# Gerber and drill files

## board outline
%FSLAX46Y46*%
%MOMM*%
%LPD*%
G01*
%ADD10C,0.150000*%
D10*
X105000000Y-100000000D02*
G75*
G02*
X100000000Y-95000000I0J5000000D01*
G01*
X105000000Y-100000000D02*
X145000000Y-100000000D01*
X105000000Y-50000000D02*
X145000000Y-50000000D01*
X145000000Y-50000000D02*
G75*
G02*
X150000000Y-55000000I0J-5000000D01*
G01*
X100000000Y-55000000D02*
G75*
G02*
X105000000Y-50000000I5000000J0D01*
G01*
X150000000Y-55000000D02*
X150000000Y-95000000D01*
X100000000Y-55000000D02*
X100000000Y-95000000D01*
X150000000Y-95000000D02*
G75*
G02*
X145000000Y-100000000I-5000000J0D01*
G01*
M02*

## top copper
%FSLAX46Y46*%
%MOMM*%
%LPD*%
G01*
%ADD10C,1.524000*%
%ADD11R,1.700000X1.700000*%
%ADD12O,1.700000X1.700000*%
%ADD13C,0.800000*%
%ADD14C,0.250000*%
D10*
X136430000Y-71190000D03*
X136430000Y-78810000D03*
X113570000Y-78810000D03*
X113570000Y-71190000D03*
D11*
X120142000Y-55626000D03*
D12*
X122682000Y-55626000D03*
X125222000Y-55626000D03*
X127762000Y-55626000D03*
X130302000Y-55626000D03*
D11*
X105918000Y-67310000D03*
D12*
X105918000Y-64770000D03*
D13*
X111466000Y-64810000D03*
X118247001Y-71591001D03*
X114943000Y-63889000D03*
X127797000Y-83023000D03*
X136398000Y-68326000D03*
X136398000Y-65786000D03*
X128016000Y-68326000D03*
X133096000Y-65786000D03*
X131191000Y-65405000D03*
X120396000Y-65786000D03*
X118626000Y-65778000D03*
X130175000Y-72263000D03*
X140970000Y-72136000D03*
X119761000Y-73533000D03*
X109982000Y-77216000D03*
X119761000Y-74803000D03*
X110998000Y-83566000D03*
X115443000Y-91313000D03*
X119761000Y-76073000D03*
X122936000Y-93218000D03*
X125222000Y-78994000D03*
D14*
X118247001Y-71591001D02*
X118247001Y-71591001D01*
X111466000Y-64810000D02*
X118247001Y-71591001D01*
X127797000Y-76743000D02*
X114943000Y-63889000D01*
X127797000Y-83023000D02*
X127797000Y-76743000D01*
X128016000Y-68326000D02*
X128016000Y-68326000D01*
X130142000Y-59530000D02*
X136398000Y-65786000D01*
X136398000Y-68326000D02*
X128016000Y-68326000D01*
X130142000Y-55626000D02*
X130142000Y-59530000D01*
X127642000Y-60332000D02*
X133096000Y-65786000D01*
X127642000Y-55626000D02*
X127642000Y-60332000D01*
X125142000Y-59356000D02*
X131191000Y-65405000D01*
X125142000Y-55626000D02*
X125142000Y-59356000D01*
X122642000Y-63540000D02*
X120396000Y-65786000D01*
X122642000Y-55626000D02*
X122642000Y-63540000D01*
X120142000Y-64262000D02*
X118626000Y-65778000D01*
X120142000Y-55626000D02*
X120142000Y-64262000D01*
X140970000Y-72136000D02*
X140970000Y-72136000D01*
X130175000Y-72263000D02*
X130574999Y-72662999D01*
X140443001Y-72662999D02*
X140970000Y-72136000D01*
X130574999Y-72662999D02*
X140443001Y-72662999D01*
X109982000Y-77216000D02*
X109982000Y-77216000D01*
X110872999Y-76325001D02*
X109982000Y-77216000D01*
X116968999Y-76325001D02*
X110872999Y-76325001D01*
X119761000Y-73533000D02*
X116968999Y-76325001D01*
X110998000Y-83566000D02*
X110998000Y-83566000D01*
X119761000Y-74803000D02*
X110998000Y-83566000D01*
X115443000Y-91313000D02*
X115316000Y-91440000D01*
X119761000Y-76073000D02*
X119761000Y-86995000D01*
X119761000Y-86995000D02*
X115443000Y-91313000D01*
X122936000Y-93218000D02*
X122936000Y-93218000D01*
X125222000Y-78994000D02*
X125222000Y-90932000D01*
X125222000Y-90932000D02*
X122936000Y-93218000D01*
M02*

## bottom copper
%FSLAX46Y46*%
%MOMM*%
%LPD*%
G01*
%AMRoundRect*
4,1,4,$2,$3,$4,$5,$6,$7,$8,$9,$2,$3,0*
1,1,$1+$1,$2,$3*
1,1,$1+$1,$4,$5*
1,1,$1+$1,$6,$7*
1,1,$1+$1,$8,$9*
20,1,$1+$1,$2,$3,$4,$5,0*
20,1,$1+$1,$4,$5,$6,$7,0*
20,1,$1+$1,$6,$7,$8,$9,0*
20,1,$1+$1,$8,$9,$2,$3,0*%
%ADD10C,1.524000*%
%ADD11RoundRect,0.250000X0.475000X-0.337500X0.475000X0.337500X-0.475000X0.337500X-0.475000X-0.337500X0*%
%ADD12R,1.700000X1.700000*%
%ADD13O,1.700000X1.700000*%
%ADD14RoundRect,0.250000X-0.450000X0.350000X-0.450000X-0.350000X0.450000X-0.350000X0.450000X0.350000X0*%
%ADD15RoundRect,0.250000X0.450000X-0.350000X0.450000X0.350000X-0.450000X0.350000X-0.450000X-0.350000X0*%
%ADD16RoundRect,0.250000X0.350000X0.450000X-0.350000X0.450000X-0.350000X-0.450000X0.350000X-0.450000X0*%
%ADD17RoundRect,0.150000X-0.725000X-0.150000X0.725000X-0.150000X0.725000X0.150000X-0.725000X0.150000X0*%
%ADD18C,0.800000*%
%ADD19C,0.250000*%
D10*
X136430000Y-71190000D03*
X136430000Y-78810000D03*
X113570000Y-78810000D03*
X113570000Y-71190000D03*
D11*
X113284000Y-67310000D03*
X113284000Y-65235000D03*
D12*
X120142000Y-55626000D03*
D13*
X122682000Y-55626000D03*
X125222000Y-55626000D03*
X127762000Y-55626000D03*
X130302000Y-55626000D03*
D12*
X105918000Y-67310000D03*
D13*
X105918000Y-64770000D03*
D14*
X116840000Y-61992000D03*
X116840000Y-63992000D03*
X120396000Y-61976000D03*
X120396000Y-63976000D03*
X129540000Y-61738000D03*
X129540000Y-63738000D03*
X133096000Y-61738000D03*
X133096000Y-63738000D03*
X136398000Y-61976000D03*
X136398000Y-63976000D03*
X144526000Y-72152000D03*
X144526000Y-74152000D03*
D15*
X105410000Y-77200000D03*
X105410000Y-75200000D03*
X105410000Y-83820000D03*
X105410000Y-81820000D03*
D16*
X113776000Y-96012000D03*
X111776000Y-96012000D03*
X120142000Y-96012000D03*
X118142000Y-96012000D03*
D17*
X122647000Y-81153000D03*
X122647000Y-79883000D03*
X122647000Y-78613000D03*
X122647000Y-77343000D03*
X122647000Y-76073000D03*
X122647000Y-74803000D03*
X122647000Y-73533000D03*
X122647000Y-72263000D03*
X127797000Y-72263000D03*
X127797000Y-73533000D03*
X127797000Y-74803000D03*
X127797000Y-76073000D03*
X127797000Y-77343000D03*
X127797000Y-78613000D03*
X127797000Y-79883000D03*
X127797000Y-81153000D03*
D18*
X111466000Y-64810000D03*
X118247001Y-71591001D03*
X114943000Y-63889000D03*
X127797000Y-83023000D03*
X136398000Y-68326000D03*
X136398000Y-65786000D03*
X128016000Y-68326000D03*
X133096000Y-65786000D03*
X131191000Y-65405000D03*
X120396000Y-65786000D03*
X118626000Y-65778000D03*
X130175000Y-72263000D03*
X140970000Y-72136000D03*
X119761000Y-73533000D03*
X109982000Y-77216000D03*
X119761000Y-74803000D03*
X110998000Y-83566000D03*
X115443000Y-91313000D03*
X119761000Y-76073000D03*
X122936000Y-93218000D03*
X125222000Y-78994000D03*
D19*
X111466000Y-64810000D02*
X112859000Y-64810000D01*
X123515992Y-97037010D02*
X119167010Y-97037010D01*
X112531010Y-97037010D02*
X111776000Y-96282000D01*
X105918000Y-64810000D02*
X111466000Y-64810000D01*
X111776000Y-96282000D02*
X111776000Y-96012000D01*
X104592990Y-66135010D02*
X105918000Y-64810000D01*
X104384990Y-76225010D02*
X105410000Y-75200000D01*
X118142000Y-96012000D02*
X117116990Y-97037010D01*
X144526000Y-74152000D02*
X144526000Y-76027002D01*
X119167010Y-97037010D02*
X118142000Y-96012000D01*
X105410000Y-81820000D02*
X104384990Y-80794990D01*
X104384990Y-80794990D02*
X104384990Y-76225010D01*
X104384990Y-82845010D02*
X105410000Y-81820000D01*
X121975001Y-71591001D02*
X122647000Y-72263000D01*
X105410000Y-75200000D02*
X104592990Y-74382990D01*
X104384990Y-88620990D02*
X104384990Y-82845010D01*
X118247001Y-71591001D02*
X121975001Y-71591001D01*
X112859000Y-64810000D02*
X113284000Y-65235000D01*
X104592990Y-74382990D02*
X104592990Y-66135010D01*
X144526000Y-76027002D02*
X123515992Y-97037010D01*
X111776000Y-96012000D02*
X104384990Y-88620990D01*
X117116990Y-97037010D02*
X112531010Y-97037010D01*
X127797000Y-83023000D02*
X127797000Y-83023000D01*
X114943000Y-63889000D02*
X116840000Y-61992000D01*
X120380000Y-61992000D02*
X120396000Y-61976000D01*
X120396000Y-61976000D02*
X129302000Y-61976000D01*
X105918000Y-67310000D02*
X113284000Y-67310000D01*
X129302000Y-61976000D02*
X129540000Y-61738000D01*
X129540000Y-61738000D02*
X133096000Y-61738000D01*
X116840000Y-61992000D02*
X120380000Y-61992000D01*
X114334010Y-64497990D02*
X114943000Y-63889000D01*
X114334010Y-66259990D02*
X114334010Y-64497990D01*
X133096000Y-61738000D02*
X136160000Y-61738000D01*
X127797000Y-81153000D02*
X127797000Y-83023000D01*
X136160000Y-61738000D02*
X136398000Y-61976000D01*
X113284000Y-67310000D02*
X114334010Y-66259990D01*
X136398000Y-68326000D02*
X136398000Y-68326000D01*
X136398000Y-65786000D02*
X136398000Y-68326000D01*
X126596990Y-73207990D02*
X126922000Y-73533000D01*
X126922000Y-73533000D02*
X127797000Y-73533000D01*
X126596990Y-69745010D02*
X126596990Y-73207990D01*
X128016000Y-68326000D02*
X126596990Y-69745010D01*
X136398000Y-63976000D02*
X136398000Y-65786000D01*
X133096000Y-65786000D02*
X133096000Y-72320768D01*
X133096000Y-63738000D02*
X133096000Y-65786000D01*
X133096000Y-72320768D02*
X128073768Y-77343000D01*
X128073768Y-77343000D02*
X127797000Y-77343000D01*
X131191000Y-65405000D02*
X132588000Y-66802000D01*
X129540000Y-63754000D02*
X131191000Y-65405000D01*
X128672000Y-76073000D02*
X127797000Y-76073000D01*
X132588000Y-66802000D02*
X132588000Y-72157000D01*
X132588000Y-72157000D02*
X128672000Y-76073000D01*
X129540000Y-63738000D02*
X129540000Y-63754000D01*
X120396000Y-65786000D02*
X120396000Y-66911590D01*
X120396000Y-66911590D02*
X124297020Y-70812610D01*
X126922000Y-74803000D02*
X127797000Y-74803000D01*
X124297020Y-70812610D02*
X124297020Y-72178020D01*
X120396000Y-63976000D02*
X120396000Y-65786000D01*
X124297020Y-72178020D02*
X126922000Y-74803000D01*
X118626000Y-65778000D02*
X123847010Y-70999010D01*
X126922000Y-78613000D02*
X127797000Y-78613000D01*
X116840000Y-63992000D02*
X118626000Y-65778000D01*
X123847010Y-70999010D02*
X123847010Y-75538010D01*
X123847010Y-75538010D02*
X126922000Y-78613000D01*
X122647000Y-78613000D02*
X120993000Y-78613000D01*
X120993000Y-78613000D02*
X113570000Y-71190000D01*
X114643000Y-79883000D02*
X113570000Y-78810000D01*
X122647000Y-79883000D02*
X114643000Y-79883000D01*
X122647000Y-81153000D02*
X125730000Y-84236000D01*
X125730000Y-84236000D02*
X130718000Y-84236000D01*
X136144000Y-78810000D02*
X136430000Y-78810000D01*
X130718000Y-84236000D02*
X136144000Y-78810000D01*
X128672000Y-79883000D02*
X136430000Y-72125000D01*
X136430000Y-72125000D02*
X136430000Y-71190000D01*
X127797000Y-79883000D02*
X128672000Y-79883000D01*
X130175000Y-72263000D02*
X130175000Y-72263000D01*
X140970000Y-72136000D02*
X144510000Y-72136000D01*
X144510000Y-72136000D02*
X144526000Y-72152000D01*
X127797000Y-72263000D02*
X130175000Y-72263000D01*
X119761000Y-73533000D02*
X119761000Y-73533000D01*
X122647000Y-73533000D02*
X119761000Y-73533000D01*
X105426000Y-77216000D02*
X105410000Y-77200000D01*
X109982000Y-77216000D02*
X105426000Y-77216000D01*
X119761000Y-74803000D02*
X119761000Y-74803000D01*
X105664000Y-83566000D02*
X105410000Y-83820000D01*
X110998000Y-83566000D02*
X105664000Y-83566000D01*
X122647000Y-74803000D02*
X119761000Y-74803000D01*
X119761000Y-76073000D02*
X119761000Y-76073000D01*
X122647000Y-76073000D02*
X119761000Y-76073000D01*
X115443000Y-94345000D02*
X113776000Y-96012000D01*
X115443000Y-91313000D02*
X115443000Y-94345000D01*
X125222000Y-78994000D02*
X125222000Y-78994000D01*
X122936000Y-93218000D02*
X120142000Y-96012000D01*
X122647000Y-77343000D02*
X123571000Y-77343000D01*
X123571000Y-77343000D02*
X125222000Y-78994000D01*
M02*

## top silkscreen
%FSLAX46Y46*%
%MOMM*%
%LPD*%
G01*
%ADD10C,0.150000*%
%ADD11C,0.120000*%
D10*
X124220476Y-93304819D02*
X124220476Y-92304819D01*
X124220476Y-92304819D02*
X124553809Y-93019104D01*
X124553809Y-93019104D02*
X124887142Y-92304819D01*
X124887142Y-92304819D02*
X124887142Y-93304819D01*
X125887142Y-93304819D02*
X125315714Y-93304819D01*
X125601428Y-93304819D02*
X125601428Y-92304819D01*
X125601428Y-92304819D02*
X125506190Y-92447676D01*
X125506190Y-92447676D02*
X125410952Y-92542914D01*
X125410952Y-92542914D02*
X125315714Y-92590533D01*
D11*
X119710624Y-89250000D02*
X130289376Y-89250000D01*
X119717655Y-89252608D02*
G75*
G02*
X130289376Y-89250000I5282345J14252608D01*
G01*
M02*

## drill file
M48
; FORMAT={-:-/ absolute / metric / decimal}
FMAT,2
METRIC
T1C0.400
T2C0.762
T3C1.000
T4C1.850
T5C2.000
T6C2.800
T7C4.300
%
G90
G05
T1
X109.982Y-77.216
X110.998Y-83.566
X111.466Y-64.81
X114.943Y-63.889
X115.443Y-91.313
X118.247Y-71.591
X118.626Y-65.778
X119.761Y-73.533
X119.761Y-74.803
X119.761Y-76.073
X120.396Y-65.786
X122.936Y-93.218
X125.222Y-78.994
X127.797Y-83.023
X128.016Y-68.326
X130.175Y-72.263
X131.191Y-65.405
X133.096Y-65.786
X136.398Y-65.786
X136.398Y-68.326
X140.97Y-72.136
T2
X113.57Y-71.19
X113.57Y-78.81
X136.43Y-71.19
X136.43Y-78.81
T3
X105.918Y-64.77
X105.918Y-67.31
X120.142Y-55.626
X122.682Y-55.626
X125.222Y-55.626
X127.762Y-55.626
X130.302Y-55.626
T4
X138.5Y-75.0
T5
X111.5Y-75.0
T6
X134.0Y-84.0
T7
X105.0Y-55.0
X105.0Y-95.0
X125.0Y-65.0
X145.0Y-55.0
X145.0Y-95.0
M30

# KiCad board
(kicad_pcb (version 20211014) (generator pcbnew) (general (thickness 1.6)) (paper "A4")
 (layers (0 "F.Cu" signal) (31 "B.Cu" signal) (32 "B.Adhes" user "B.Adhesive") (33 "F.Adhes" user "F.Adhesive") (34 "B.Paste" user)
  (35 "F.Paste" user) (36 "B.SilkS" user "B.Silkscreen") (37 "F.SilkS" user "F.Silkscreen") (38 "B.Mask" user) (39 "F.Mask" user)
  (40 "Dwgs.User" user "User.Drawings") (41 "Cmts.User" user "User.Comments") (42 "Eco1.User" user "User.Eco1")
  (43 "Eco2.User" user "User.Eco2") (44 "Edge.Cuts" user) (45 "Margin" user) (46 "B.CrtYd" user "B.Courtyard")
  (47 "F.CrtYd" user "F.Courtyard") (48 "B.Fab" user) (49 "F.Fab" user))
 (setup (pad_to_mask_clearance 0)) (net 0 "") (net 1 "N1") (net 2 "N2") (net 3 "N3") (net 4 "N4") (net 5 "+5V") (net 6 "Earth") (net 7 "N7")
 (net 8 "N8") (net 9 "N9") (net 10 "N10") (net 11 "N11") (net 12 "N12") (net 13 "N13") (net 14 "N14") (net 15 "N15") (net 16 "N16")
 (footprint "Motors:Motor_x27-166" (layer "F.Cu") (at 125 75)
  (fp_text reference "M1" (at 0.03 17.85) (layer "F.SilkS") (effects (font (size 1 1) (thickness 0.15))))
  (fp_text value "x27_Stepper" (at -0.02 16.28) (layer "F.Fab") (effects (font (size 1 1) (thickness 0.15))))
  (fp_line (start -5.289376 14.25) (end 5.289376 14.25) (layer "F.SilkS") (width 0.12))
  (fp_arc (start -5.282345 14.252608) (mid -0.00375 -15.2) (end 5.289376 14.25) (layer "F.SilkS") (width 0.12))
  (pad "" np_thru_hole circle locked (at 13.5 0) (size 1.85 1.85) (drill 1.85) (layers *.Cu *.Mask))
  (pad "" np_thru_hole circle locked (at 0 -10) (size 4.3 4.3) (drill 4.3) (layers *.Cu *.Mask))
  (pad "" np_thru_hole circle locked (at 9 9) (size 2.8 2.8) (drill 2.8) (layers *.Cu *.Mask))
  (pad "" np_thru_hole circle locked (at -13.5 0) (size 2 2) (drill 2) (layers *.Cu *.Mask))
  (pad "1" thru_hole circle locked (at 11.43 -3.81) (size 1.524 1.524) (drill 0.762) (layers *.Cu *.Mask) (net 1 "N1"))
  (pad "2" thru_hole circle locked (at 11.43 3.81) (size 1.524 1.524) (drill 0.762) (layers *.Cu *.Mask) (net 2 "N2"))
  (pad "3" thru_hole circle locked (at -11.43 3.81) (size 1.524 1.524) (drill 0.762) (layers *.Cu *.Mask) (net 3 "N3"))
  (pad "4" thru_hole circle locked (at -11.43 -3.81) (size 1.524 1.524) (drill 0.762) (layers *.Cu *.Mask) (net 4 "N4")))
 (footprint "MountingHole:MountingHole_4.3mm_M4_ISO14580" (layer "F.Cu") (at 105 55)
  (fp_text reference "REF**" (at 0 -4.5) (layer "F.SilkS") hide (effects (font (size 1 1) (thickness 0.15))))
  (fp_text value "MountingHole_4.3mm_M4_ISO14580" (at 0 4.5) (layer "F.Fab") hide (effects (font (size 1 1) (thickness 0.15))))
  (pad "" np_thru_hole circle locked (at 0 0) (size 4.3 4.3) (drill 4.3) (layers *.Cu *.Mask)))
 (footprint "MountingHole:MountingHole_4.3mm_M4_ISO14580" (layer "F.Cu") (at 145 55)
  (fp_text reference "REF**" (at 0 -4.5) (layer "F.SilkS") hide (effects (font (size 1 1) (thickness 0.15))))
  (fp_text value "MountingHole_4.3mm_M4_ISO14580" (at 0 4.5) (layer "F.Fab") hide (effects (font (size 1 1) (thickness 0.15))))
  (pad "" np_thru_hole circle locked (at 0 0) (size 4.3 4.3) (drill 4.3) (layers *.Cu *.Mask)))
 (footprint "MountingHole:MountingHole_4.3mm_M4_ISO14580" (layer "F.Cu") (at 105 95)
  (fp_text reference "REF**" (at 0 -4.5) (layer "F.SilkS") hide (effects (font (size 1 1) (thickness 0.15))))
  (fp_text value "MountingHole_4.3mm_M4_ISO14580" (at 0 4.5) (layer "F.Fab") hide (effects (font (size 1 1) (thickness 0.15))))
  (pad "" np_thru_hole circle locked (at 0 0) (size 4.3 4.3) (drill 4.3) (layers *.Cu *.Mask)))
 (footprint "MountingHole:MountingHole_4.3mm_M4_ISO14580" (layer "F.Cu") (at 145 95)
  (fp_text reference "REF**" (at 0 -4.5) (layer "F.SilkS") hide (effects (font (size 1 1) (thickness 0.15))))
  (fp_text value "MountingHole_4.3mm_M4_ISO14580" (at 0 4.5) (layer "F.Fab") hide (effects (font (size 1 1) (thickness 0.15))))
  (pad "" np_thru_hole circle locked (at 0 0) (size 4.3 4.3) (drill 4.3) (layers *.Cu *.Mask)))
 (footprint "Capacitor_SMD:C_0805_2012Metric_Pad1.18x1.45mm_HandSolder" (layer "B.Cu") (at 113.284 66.2725 90)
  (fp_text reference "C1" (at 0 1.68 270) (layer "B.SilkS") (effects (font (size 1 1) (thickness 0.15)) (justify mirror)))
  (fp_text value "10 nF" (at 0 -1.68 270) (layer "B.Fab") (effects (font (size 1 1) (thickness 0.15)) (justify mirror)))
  (pad "1" smd roundrect locked (at -1.0375 0 90) (size 1.175 1.45) (layers "B.Cu" "B.Paste" "B.Mask") (roundrect_rratio 0.2127659574)
   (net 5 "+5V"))
  (pad "2" smd roundrect locked (at 1.0375 0 90) (size 1.175 1.45) (layers "B.Cu" "B.Paste" "B.Mask") (roundrect_rratio 0.2127659574)
   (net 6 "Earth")))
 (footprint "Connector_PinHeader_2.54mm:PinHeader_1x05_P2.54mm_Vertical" (layer "B.Cu") (at 120.142 55.626 -90)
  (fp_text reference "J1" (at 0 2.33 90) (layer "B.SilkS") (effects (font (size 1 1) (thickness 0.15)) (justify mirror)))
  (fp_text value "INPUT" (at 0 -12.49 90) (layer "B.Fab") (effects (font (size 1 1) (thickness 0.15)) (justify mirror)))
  (pad "1" thru_hole rect (at 0 0 270) (size 1.7 1.7) (drill 1) (layers *.Cu *.Mask) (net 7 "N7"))
  (pad "2" thru_hole oval (at 0 -2.54 270) (size 1.7 1.7) (drill 1) (layers *.Cu *.Mask) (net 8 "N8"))
  (pad "3" thru_hole oval (at 0 -5.08 270) (size 1.7 1.7) (drill 1) (layers *.Cu *.Mask) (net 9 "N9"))
  (pad "4" thru_hole oval (at 0 -7.62 270) (size 1.7 1.7) (drill 1) (layers *.Cu *.Mask) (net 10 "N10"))
  (pad "5" thru_hole oval (at 0 -10.16 270) (size 1.7 1.7) (drill 1) (layers *.Cu *.Mask) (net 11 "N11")))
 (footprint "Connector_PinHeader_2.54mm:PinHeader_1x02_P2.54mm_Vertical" (layer "B.Cu") (at 105.918 67.31)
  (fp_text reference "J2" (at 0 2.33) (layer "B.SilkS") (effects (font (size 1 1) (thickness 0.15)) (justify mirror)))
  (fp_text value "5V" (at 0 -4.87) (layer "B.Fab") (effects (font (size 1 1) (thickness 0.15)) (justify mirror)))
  (pad "1" thru_hole rect (at 0 0) (size 1.7 1.7) (drill 1) (layers *.Cu *.Mask) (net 5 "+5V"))
  (pad "2" thru_hole oval (at 0 -2.54) (size 1.7 1.7) (drill 1) (layers *.Cu *.Mask) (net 6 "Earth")))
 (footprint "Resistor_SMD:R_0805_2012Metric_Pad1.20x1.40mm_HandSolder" (layer "B.Cu") (at 116.84 62.992 -90)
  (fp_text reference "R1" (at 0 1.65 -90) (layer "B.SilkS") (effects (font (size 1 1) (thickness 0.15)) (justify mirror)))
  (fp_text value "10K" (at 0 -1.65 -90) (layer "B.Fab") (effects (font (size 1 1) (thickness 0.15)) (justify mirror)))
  (pad "1" smd roundrect locked (at -1 0 270) (size 1.2 1.4) (layers "B.Cu" "B.Paste" "B.Mask") (roundrect_rratio 0.2083333333)
   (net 5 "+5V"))
  (pad "2" smd roundrect locked (at 1 0 270) (size 1.2 1.4) (layers "B.Cu" "B.Paste" "B.Mask") (roundrect_rratio 0.2083333333) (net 7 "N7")))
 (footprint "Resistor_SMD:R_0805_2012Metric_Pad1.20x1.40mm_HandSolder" (layer "B.Cu") (at 120.396 62.976 -90)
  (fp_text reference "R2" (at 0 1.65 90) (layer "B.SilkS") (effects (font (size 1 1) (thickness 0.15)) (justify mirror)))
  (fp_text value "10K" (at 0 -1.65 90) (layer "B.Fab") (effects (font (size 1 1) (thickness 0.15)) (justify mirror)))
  (pad "1" smd roundrect locked (at -1 0 270) (size 1.2 1.4) (layers "B.Cu" "B.Paste" "B.Mask") (roundrect_rratio 0.2083333333)
   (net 5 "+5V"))
  (pad "2" smd roundrect locked (at 1 0 270) (size 1.2 1.4) (layers "B.Cu" "B.Paste" "B.Mask") (roundrect_rratio 0.2083333333) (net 8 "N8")))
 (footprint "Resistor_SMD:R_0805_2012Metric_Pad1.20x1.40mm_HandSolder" (layer "B.Cu") (at 129.54 62.738 -90)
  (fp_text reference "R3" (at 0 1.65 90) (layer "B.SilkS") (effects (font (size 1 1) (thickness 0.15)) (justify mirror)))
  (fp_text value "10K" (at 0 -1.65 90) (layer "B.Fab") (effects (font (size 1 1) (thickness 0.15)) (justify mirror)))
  (pad "1" smd roundrect locked (at -1 0 270) (size 1.2 1.4) (layers "B.Cu" "B.Paste" "B.Mask") (roundrect_rratio 0.2083333333)
   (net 5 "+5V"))
  (pad "2" smd roundrect locked (at 1 0 270) (size 1.2 1.4) (layers "B.Cu" "B.Paste" "B.Mask") (roundrect_rratio 0.2083333333) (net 9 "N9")))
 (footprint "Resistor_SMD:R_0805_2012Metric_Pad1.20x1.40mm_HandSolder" (layer "B.Cu") (at 133.096 62.738 -90)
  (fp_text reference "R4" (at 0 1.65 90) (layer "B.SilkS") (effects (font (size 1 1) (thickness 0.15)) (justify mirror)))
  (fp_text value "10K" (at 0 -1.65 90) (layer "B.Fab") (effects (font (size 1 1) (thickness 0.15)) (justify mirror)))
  (pad "1" smd roundrect locked (at -1 0 270) (size 1.2 1.4) (layers "B.Cu" "B.Paste" "B.Mask") (roundrect_rratio 0.2083333333)
   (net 5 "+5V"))
  (pad "2" smd roundrect locked (at 1 0 270) (size 1.2 1.4) (layers "B.Cu" "B.Paste" "B.Mask") (roundrect_rratio 0.2083333333)
   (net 10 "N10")))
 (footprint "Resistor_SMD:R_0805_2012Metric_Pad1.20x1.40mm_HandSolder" (layer "B.Cu") (at 136.398 62.976 -90)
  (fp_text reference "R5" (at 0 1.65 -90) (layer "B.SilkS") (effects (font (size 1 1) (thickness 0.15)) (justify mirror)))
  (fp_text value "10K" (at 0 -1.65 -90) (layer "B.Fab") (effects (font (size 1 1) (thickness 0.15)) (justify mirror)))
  (pad "1" smd roundrect locked (at -1 0 270) (size 1.2 1.4) (layers "B.Cu" "B.Paste" "B.Mask") (roundrect_rratio 0.2083333333)
   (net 5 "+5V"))
  (pad "2" smd roundrect locked (at 1 0 270) (size 1.2 1.4) (layers "B.Cu" "B.Paste" "B.Mask") (roundrect_rratio 0.2083333333)
   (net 11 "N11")))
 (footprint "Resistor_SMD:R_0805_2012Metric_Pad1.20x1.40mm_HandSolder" (layer "B.Cu") (at 144.526 73.152 -90)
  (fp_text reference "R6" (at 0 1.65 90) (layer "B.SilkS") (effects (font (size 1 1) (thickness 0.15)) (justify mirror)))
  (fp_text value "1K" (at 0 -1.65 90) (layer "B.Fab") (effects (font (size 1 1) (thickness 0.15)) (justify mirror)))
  (pad "1" smd roundrect locked (at -1 0 270) (size 1.2 1.4) (layers "B.Cu" "B.Paste" "B.Mask") (roundrect_rratio 0.2083333333)
   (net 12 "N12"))
  (pad "2" smd roundrect locked (at 1 0 270) (size 1.2 1.4) (layers "B.Cu" "B.Paste" "B.Mask") (roundrect_rratio 0.2083333333)
   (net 6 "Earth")))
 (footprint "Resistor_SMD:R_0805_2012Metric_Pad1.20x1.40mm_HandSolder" (layer "B.Cu") (at 105.41 76.2 90)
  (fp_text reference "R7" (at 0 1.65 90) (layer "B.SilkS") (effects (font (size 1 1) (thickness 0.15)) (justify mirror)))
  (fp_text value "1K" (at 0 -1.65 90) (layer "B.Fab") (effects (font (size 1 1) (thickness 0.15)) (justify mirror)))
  (pad "1" smd roundrect locked (at -1 0 90) (size 1.2 1.4) (layers "B.Cu" "B.Paste" "B.Mask") (roundrect_rratio 0.2083333333)
   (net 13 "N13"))
  (pad "2" smd roundrect locked (at 1 0 90) (size 1.2 1.4) (layers "B.Cu" "B.Paste" "B.Mask") (roundrect_rratio 0.2083333333)
   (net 6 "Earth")))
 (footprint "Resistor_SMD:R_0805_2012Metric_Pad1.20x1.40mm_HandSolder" (layer "B.Cu") (at 105.41 82.82 90)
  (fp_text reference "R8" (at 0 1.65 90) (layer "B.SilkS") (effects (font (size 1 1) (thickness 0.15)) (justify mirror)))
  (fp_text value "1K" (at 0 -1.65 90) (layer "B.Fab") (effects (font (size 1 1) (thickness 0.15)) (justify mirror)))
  (pad "1" smd roundrect locked (at -1 0 90) (size 1.2 1.4) (layers "B.Cu" "B.Paste" "B.Mask") (roundrect_rratio 0.2083333333)
   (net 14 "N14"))
  (pad "2" smd roundrect locked (at 1 0 90) (size 1.2 1.4) (layers "B.Cu" "B.Paste" "B.Mask") (roundrect_rratio 0.2083333333)
   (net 6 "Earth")))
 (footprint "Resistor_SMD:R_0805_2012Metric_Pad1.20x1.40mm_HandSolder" (layer "B.Cu") (at 112.776 96.012 180)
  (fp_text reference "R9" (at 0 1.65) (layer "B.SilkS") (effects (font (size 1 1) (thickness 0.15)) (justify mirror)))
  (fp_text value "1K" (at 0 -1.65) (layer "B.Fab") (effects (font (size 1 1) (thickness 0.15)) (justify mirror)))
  (pad "1" smd roundrect locked (at -1 0 180) (size 1.2 1.4) (layers "B.Cu" "B.Paste" "B.Mask") (roundrect_rratio 0.2083333333)
   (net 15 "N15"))
  (pad "2" smd roundrect locked (at 1 0 180) (size 1.2 1.4) (layers "B.Cu" "B.Paste" "B.Mask") (roundrect_rratio 0.2083333333)
   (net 6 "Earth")))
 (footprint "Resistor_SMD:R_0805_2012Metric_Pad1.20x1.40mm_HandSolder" (layer "B.Cu") (at 119.142 96.012 180)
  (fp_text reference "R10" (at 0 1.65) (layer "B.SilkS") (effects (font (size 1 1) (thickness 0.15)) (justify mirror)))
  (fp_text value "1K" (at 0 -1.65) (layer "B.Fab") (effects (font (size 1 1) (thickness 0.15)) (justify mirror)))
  (pad "1" smd roundrect locked (at -1 0 180) (size 1.2 1.4) (layers "B.Cu" "B.Paste" "B.Mask") (roundrect_rratio 0.2083333333)
   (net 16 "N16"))
  (pad "2" smd roundrect locked (at 1 0 180) (size 1.2 1.4) (layers "B.Cu" "B.Paste" "B.Mask") (roundrect_rratio 0.2083333333)
   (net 6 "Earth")))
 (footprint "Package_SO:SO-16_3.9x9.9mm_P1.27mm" (layer "B.Cu") (at 125.222 76.708)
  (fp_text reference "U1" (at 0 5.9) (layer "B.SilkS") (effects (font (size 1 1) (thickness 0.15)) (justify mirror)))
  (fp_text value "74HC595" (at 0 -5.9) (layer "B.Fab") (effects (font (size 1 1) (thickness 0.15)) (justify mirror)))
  (pad "1" smd roundrect locked (at -2.575 4.445) (size 1.75 0.6) (layers "B.Cu" "B.Paste" "B.Mask") (roundrect_rratio 0.25) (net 2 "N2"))
  (pad "2" smd roundrect locked (at -2.575 3.175) (size 1.75 0.6) (layers "B.Cu" "B.Paste" "B.Mask") (roundrect_rratio 0.25) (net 3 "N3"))
  (pad "3" smd roundrect locked (at -2.575 1.905) (size 1.75 0.6) (layers "B.Cu" "B.Paste" "B.Mask") (roundrect_rratio 0.25) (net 4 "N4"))
  (pad "4" smd roundrect locked (at -2.575 0.635) (size 1.75 0.6) (layers "B.Cu" "B.Paste" "B.Mask") (roundrect_rratio 0.25) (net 16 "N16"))
  (pad "5" smd roundrect locked (at -2.575 -0.635) (size 1.75 0.6) (layers "B.Cu" "B.Paste" "B.Mask") (roundrect_rratio 0.25) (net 15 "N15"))
  (pad "6" smd roundrect locked (at -2.575 -1.905) (size 1.75 0.6) (layers "B.Cu" "B.Paste" "B.Mask") (roundrect_rratio 0.25) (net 14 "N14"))
  (pad "7" smd roundrect locked (at -2.575 -3.175) (size 1.75 0.6) (layers "B.Cu" "B.Paste" "B.Mask") (roundrect_rratio 0.25) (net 13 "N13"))
  (pad "8" smd roundrect locked (at -2.575 -4.445) (size 1.75 0.6) (layers "B.Cu" "B.Paste" "B.Mask") (roundrect_rratio 0.25)
   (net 6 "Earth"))
  (pad "9" smd roundrect locked (at 2.575 -4.445) (size 1.75 0.6) (layers "B.Cu" "B.Paste" "B.Mask") (roundrect_rratio 0.25) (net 12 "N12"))
  (pad "10" smd roundrect locked (at 2.575 -3.175) (size 1.75 0.6) (layers "B.Cu" "B.Paste" "B.Mask") (roundrect_rratio 0.25) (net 11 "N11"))
  (pad "11" smd roundrect locked (at 2.575 -1.905) (size 1.75 0.6) (layers "B.Cu" "B.Paste" "B.Mask") (roundrect_rratio 0.25) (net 8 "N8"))
  (pad "12" smd roundrect locked (at 2.575 -0.635) (size 1.75 0.6) (layers "B.Cu" "B.Paste" "B.Mask") (roundrect_rratio 0.25) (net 9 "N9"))
  (pad "13" smd roundrect locked (at 2.575 0.635) (size 1.75 0.6) (layers "B.Cu" "B.Paste" "B.Mask") (roundrect_rratio 0.25) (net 10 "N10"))
  (pad "14" smd roundrect locked (at 2.575 1.905) (size 1.75 0.6) (layers "B.Cu" "B.Paste" "B.Mask") (roundrect_rratio 0.25) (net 7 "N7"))
  (pad "15" smd roundrect locked (at 2.575 3.175) (size 1.75 0.6) (layers "B.Cu" "B.Paste" "B.Mask") (roundrect_rratio 0.25) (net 1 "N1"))
  (pad "16" smd roundrect locked (at 2.575 4.445) (size 1.75 0.6) (layers "B.Cu" "B.Paste" "B.Mask") (roundrect_rratio 0.25) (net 5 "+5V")))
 (gr_arc (start 105 100) (mid 101.464466 98.535534) (end 100 95) (layer "Edge.Cuts") (width 0.15))
 (gr_line (start 105 100) (end 145 100) (layer "Edge.Cuts") (width 0.15))
 (gr_line (start 105 50) (end 145 50) (layer "Edge.Cuts") (width 0.15))
 (gr_arc (start 145 50) (mid 148.535534 51.464466) (end 150 55) (layer "Edge.Cuts") (width 0.15))
 (gr_arc (start 100 55) (mid 101.464466 51.464466) (end 105 50) (layer "Edge.Cuts") (width 0.15))
 (gr_line (start 150 55) (end 150 95) (layer "Edge.Cuts") (width 0.15))
 (gr_line (start 100 55) (end 100 95) (layer "Edge.Cuts") (width 0.15))
 (gr_arc (start 150 95) (mid 148.535534 98.535534) (end 145 100) (layer "Edge.Cuts") (width 0.15))
 (segment (start 118.247001 71.591001) (end 118.247001 71.591001) (width 0.25) (layer "F.Cu") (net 6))
 (segment (start 111.466 64.81) (end 118.247001 71.591001) (width 0.25) (layer "F.Cu") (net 6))
 (via (at 111.466 64.81) (size 0.8) (drill 0.4) (layers "F.Cu" "B.Cu") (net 6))
 (via (at 118.247001 71.591001) (size 0.8) (drill 0.4) (layers "F.Cu" "B.Cu") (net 6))
 (segment (start 111.466 64.81) (end 112.859 64.81) (width 0.25) (layer "B.Cu") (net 6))
 (segment (start 123.515992 97.03701) (end 119.16701 97.03701) (width 0.25) (layer "B.Cu") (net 6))
 (segment (start 112.53101 97.03701) (end 111.776 96.282) (width 0.25) (layer "B.Cu") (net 6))
 (segment (start 105.918 64.81) (end 111.466 64.81) (width 0.25) (layer "B.Cu") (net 6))
 (segment (start 111.776 96.282) (end 111.776 96.012) (width 0.25) (layer "B.Cu") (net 6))
 (segment (start 104.59299 66.13501) (end 105.918 64.81) (width 0.25) (layer "B.Cu") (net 6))
 (segment (start 104.38499 76.22501) (end 105.41 75.2) (width 0.25) (layer "B.Cu") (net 6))
 (segment (start 118.142 96.012) (end 117.11699 97.03701) (width 0.25) (layer "B.Cu") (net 6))
 (segment (start 144.526 74.152) (end 144.526 76.027002) (width 0.25) (layer "B.Cu") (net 6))
 (segment (start 119.16701 97.03701) (end 118.142 96.012) (width 0.25) (layer "B.Cu") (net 6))
 (segment (start 105.41 81.82) (end 104.38499 80.79499) (width 0.25) (layer "B.Cu") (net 6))
 (segment (start 104.38499 80.79499) (end 104.38499 76.22501) (width 0.25) (layer "B.Cu") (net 6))
 (segment (start 104.38499 82.84501) (end 105.41 81.82) (width 0.25) (layer "B.Cu") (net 6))
 (segment (start 121.975001 71.591001) (end 122.647 72.263) (width 0.25) (layer "B.Cu") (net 6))
 (segment (start 105.41 75.2) (end 104.59299 74.38299) (width 0.25) (layer "B.Cu") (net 6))
 (segment (start 104.38499 88.62099) (end 104.38499 82.84501) (width 0.25) (layer "B.Cu") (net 6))
 (segment (start 118.247001 71.591001) (end 121.975001 71.591001) (width 0.25) (layer "B.Cu") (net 6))
 (segment (start 112.859 64.81) (end 113.284 65.235) (width 0.25) (layer "B.Cu") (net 6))
 (segment (start 104.59299 74.38299) (end 104.59299 66.13501) (width 0.25) (layer "B.Cu") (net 6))
 (segment (start 144.526 76.027002) (end 123.515992 97.03701) (width 0.25) (layer "B.Cu") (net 6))
 (segment (start 111.776 96.012) (end 104.38499 88.62099) (width 0.25) (layer "B.Cu") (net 6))
 (segment (start 117.11699 97.03701) (end 112.53101 97.03701) (width 0.25) (layer "B.Cu") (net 6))
 (segment (start 127.797 76.743) (end 114.943 63.889) (width 0.25) (layer "F.Cu") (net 5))
 (segment (start 127.797 83.023) (end 127.797 76.743) (width 0.25) (layer "F.Cu") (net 5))
 (via (at 114.943 63.889) (size 0.8) (drill 0.4) (layers "F.Cu" "B.Cu") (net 5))
 (via (at 127.797 83.023) (size 0.8) (drill 0.4) (layers "F.Cu" "B.Cu") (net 5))
 (segment (start 127.797 83.023) (end 127.797 83.023) (width 0.25) (layer "B.Cu") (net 5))
 (segment (start 114.943 63.889) (end 116.84 61.992) (width 0.25) (layer "B.Cu") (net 5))
 (segment (start 120.38 61.992) (end 120.396 61.976) (width 0.25) (layer "B.Cu") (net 5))
 (segment (start 120.396 61.976) (end 129.302 61.976) (width 0.25) (layer "B.Cu") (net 5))
 (segment (start 105.918 67.31) (end 113.284 67.31) (width 0.25) (layer "B.Cu") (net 5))
 (segment (start 129.302 61.976) (end 129.54 61.738) (width 0.25) (layer "B.Cu") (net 5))
 (segment (start 129.54 61.738) (end 133.096 61.738) (width 0.25) (layer "B.Cu") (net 5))
 (segment (start 116.84 61.992) (end 120.38 61.992) (width 0.25) (layer "B.Cu") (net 5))
 (segment (start 114.33401 64.49799) (end 114.943 63.889) (width 0.25) (layer "B.Cu") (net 5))
 (segment (start 114.33401 66.25999) (end 114.33401 64.49799) (width 0.25) (layer "B.Cu") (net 5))
 (segment (start 133.096 61.738) (end 136.16 61.738) (width 0.25) (layer "B.Cu") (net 5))
 (segment (start 127.797 81.153) (end 127.797 83.023) (width 0.25) (layer "B.Cu") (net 5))
 (segment (start 136.16 61.738) (end 136.398 61.976) (width 0.25) (layer "B.Cu") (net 5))
 (segment (start 113.284 67.31) (end 114.33401 66.25999) (width 0.25) (layer "B.Cu") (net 5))
 (segment (start 128.016 68.326) (end 128.016 68.326) (width 0.25) (layer "F.Cu") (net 11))
 (segment (start 130.142 59.53) (end 136.398 65.786) (width 0.25) (layer "F.Cu") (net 11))
 (segment (start 136.398 68.326) (end 128.016 68.326) (width 0.25) (layer "F.Cu") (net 11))
 (segment (start 130.142 55.626) (end 130.142 59.53) (width 0.25) (layer "F.Cu") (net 11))
 (via (at 136.398 68.326) (size 0.8) (drill 0.4) (layers "F.Cu" "B.Cu") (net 11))
 (via (at 136.398 65.786) (size 0.8) (drill 0.4) (layers "F.Cu" "B.Cu") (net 11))
 (via (at 128.016 68.326) (size 0.8) (drill 0.4) (layers "F.Cu" "B.Cu") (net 11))
 (segment (start 136.398 68.326) (end 136.398 68.326) (width 0.25) (layer "B.Cu") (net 11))
 (segment (start 136.398 65.786) (end 136.398 68.326) (width 0.25) (layer "B.Cu") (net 11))
 (segment (start 126.59699 73.20799) (end 126.922 73.533) (width 0.25) (layer "B.Cu") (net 11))
 (segment (start 126.922 73.533) (end 127.797 73.533) (width 0.25) (layer "B.Cu") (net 11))
 (segment (start 126.59699 69.74501) (end 126.59699 73.20799) (width 0.25) (layer "B.Cu") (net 11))
 (segment (start 128.016 68.326) (end 126.59699 69.74501) (width 0.25) (layer "B.Cu") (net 11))
 (segment (start 136.398 63.976) (end 136.398 65.786) (width 0.25) (layer "B.Cu") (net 11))
 (segment (start 127.642 60.332) (end 133.096 65.786) (width 0.25) (layer "F.Cu") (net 10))
 (segment (start 127.642 55.626) (end 127.642 60.332) (width 0.25) (layer "F.Cu") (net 10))
 (via (at 133.096 65.786) (size 0.8) (drill 0.4) (layers "F.Cu" "B.Cu") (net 10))
 (segment (start 133.096 65.786) (end 133.096 72.320768) (width 0.25) (layer "B.Cu") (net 10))
 (segment (start 133.096 63.738) (end 133.096 65.786) (width 0.25) (layer "B.Cu") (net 10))
 (segment (start 133.096 72.320768) (end 128.073768 77.343) (width 0.25) (layer "B.Cu") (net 10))
 (segment (start 128.073768 77.343) (end 127.797 77.343) (width 0.25) (layer "B.Cu") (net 10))
 (segment (start 125.142 59.356) (end 131.191 65.405) (width 0.25) (layer "F.Cu") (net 9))
 (segment (start 125.142 55.626) (end 125.142 59.356) (width 0.25) (layer "F.Cu") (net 9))
 (via (at 131.191 65.405) (size 0.8) (drill 0.4) (layers "F.Cu" "B.Cu") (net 9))
 (segment (start 131.191 65.405) (end 132.588 66.802) (width 0.25) (layer "B.Cu") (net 9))
 (segment (start 129.54 63.754) (end 131.191 65.405) (width 0.25) (layer "B.Cu") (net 9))
 (segment (start 128.672 76.073) (end 127.797 76.073) (width 0.25) (layer "B.Cu") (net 9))
 (segment (start 132.588 66.802) (end 132.588 72.157) (width 0.25) (layer "B.Cu") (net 9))
 (segment (start 132.588 72.157) (end 128.672 76.073) (width 0.25) (layer "B.Cu") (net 9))
 (segment (start 129.54 63.738) (end 129.54 63.754) (width 0.25) (layer "B.Cu") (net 9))
 (segment (start 122.642 63.54) (end 120.396 65.786) (width 0.25) (layer "F.Cu") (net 8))
 (segment (start 122.642 55.626) (end 122.642 63.54) (width 0.25) (layer "F.Cu") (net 8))
 (via (at 120.396 65.786) (size 0.8) (drill 0.4) (layers "F.Cu" "B.Cu") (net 8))
 (segment (start 120.396 65.786) (end 120.396 66.91159) (width 0.25) (layer "B.Cu") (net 8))
 (segment (start 120.396 66.91159) (end 124.29702 70.81261) (width 0.25) (layer "B.Cu") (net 8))
 (segment (start 126.922 74.803) (end 127.797 74.803) (width 0.25) (layer "B.Cu") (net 8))
 (segment (start 124.29702 70.81261) (end 124.29702 72.17802) (width 0.25) (layer "B.Cu") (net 8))
 (segment (start 120.396 63.976) (end 120.396 65.786) (width 0.25) (layer "B.Cu") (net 8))
 (segment (start 124.29702 72.17802) (end 126.922 74.803) (width 0.25) (layer "B.Cu") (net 8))
 (segment (start 120.142 64.262) (end 118.626 65.778) (width 0.25) (layer "F.Cu") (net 7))
 (segment (start 120.142 55.626) (end 120.142 64.262) (width 0.25) (layer "F.Cu") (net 7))
 (via (at 118.626 65.778) (size 0.8) (drill 0.4) (layers "F.Cu" "B.Cu") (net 7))
 (segment (start 118.626 65.778) (end 123.84701 70.99901) (width 0.25) (layer "B.Cu") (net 7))
 (segment (start 126.922 78.613) (end 127.797 78.613) (width 0.25) (layer "B.Cu") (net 7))
 (segment (start 116.84 63.992) (end 118.626 65.778) (width 0.25) (layer "B.Cu") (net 7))
 (segment (start 123.84701 70.99901) (end 123.84701 75.53801) (width 0.25) (layer "B.Cu") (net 7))
 (segment (start 123.84701 75.53801) (end 126.922 78.613) (width 0.25) (layer "B.Cu") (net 7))
 (segment (start 122.647 78.613) (end 120.993 78.613) (width 0.25) (layer "B.Cu") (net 4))
 (segment (start 120.993 78.613) (end 113.57 71.19) (width 0.25) (layer "B.Cu") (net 4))
 (segment (start 114.643 79.883) (end 113.57 78.81) (width 0.25) (layer "B.Cu") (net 3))
 (segment (start 122.647 79.883) (end 114.643 79.883) (width 0.25) (layer "B.Cu") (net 3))
 (segment (start 122.647 81.153) (end 125.73 84.236) (width 0.25) (layer "B.Cu") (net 2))
 (segment (start 125.73 84.236) (end 130.718 84.236) (width 0.25) (layer "B.Cu") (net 2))
 (segment (start 136.144 78.81) (end 136.43 78.81) (width 0.25) (layer "B.Cu") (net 2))
 (segment (start 130.718 84.236) (end 136.144 78.81) (width 0.25) (layer "B.Cu") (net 2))
 (segment (start 128.672 79.883) (end 136.43 72.125) (width 0.25) (layer "B.Cu") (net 1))
 (segment (start 136.43 72.125) (end 136.43 71.19) (width 0.25) (layer "B.Cu") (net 1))
 (segment (start 127.797 79.883) (end 128.672 79.883) (width 0.25) (layer "B.Cu") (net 1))
 (segment (start 140.97 72.136) (end 140.97 72.136) (width 0.25) (layer "F.Cu") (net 12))
 (segment (start 130.175 72.263) (end 130.574999 72.662999) (width 0.25) (layer "F.Cu") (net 12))
 (segment (start 140.443001 72.662999) (end 140.97 72.136) (width 0.25) (layer "F.Cu") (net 12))
 (segment (start 130.574999 72.662999) (end 140.443001 72.662999) (width 0.25) (layer "F.Cu") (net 12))
 (via (at 130.175 72.263) (size 0.8) (drill 0.4) (layers "F.Cu" "B.Cu") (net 12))
 (via (at 140.97 72.136) (size 0.8) (drill 0.4) (layers "F.Cu" "B.Cu") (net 12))
 (segment (start 130.175 72.263) (end 130.175 72.263) (width 0.25) (layer "B.Cu") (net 12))
 (segment (start 140.97 72.136) (end 144.51 72.136) (width 0.25) (layer "B.Cu") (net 12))
 (segment (start 144.51 72.136) (end 144.526 72.152) (width 0.25) (layer "B.Cu") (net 12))
 (segment (start 127.797 72.263) (end 130.175 72.263) (width 0.25) (layer "B.Cu") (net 12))
 (segment (start 109.982 77.216) (end 109.982 77.216) (width 0.25) (layer "F.Cu") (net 13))
 (segment (start 110.872999 76.325001) (end 109.982 77.216) (width 0.25) (layer "F.Cu") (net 13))
 (segment (start 116.968999 76.325001) (end 110.872999 76.325001) (width 0.25) (layer "F.Cu") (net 13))
 (segment (start 119.761 73.533) (end 116.968999 76.325001) (width 0.25) (layer "F.Cu") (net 13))
 (via (at 119.761 73.533) (size 0.8) (drill 0.4) (layers "F.Cu" "B.Cu") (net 13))
 (via (at 109.982 77.216) (size 0.8) (drill 0.4) (layers "F.Cu" "B.Cu") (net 13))
 (segment (start 119.761 73.533) (end 119.761 73.533) (width 0.25) (layer "B.Cu") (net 13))
 (segment (start 122.647 73.533) (end 119.761 73.533) (width 0.25) (layer "B.Cu") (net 13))
 (segment (start 105.426 77.216) (end 105.41 77.2) (width 0.25) (layer "B.Cu") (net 13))
 (segment (start 109.982 77.216) (end 105.426 77.216) (width 0.25) (layer "B.Cu") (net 13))
 (segment (start 110.998 83.566) (end 110.998 83.566) (width 0.25) (layer "F.Cu") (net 14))
 (segment (start 119.761 74.803) (end 110.998 83.566) (width 0.25) (layer "F.Cu") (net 14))
 (via (at 119.761 74.803) (size 0.8) (drill 0.4) (layers "F.Cu" "B.Cu") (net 14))
 (via (at 110.998 83.566) (size 0.8) (drill 0.4) (layers "F.Cu" "B.Cu") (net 14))
 (segment (start 119.761 74.803) (end 119.761 74.803) (width 0.25) (layer "B.Cu") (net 14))
 (segment (start 105.664 83.566) (end 105.41 83.82) (width 0.25) (layer "B.Cu") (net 14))
 (segment (start 110.998 83.566) (end 105.664 83.566) (width 0.25) (layer "B.Cu") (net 14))
 (segment (start 122.647 74.803) (end 119.761 74.803) (width 0.25) (layer "B.Cu") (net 14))
 (segment (start 115.443 91.313) (end 115.316 91.44) (width 0.25) (layer "F.Cu") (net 15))
 (segment (start 119.761 76.073) (end 119.761 86.995) (width 0.25) (layer "F.Cu") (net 15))
 (segment (start 119.761 86.995) (end 115.443 91.313) (width 0.25) (layer "F.Cu") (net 15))
 (via (at 115.443 91.313) (size 0.8) (drill 0.4) (layers "F.Cu" "B.Cu") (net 15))
 (via (at 119.761 76.073) (size 0.8) (drill 0.4) (layers "F.Cu" "B.Cu") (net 15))
 (segment (start 119.761 76.073) (end 119.761 76.073) (width 0.25) (layer "B.Cu") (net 15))
 (segment (start 122.647 76.073) (end 119.761 76.073) (width 0.25) (layer "B.Cu") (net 15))
 (segment (start 115.443 94.345) (end 113.776 96.012) (width 0.25) (layer "B.Cu") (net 15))
 (segment (start 115.443 91.313) (end 115.443 94.345) (width 0.25) (layer "B.Cu") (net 15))
 (segment (start 122.936 93.218) (end 122.936 93.218) (width 0.25) (layer "F.Cu") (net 16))
 (segment (start 125.222 78.994) (end 125.222 90.932) (width 0.25) (layer "F.Cu") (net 16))
 (segment (start 125.222 90.932) (end 122.936 93.218) (width 0.25) (layer "F.Cu") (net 16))
 (via (at 122.936 93.218) (size 0.8) (drill 0.4) (layers "F.Cu" "B.Cu") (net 16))
 (via (at 125.222 78.994) (size 0.8) (drill 0.4) (layers "F.Cu" "B.Cu") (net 16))
 (segment (start 125.222 78.994) (end 125.222 78.994) (width 0.25) (layer "B.Cu") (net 16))
 (segment (start 122.936 93.218) (end 120.142 96.012) (width 0.25) (layer "B.Cu") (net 16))
 (segment (start 122.647 77.343) (end 123.571 77.343) (width 0.25) (layer "B.Cu") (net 16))
 (segment (start 123.571 77.343) (end 125.222 78.994) (width 0.25) (layer "B.Cu") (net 16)))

